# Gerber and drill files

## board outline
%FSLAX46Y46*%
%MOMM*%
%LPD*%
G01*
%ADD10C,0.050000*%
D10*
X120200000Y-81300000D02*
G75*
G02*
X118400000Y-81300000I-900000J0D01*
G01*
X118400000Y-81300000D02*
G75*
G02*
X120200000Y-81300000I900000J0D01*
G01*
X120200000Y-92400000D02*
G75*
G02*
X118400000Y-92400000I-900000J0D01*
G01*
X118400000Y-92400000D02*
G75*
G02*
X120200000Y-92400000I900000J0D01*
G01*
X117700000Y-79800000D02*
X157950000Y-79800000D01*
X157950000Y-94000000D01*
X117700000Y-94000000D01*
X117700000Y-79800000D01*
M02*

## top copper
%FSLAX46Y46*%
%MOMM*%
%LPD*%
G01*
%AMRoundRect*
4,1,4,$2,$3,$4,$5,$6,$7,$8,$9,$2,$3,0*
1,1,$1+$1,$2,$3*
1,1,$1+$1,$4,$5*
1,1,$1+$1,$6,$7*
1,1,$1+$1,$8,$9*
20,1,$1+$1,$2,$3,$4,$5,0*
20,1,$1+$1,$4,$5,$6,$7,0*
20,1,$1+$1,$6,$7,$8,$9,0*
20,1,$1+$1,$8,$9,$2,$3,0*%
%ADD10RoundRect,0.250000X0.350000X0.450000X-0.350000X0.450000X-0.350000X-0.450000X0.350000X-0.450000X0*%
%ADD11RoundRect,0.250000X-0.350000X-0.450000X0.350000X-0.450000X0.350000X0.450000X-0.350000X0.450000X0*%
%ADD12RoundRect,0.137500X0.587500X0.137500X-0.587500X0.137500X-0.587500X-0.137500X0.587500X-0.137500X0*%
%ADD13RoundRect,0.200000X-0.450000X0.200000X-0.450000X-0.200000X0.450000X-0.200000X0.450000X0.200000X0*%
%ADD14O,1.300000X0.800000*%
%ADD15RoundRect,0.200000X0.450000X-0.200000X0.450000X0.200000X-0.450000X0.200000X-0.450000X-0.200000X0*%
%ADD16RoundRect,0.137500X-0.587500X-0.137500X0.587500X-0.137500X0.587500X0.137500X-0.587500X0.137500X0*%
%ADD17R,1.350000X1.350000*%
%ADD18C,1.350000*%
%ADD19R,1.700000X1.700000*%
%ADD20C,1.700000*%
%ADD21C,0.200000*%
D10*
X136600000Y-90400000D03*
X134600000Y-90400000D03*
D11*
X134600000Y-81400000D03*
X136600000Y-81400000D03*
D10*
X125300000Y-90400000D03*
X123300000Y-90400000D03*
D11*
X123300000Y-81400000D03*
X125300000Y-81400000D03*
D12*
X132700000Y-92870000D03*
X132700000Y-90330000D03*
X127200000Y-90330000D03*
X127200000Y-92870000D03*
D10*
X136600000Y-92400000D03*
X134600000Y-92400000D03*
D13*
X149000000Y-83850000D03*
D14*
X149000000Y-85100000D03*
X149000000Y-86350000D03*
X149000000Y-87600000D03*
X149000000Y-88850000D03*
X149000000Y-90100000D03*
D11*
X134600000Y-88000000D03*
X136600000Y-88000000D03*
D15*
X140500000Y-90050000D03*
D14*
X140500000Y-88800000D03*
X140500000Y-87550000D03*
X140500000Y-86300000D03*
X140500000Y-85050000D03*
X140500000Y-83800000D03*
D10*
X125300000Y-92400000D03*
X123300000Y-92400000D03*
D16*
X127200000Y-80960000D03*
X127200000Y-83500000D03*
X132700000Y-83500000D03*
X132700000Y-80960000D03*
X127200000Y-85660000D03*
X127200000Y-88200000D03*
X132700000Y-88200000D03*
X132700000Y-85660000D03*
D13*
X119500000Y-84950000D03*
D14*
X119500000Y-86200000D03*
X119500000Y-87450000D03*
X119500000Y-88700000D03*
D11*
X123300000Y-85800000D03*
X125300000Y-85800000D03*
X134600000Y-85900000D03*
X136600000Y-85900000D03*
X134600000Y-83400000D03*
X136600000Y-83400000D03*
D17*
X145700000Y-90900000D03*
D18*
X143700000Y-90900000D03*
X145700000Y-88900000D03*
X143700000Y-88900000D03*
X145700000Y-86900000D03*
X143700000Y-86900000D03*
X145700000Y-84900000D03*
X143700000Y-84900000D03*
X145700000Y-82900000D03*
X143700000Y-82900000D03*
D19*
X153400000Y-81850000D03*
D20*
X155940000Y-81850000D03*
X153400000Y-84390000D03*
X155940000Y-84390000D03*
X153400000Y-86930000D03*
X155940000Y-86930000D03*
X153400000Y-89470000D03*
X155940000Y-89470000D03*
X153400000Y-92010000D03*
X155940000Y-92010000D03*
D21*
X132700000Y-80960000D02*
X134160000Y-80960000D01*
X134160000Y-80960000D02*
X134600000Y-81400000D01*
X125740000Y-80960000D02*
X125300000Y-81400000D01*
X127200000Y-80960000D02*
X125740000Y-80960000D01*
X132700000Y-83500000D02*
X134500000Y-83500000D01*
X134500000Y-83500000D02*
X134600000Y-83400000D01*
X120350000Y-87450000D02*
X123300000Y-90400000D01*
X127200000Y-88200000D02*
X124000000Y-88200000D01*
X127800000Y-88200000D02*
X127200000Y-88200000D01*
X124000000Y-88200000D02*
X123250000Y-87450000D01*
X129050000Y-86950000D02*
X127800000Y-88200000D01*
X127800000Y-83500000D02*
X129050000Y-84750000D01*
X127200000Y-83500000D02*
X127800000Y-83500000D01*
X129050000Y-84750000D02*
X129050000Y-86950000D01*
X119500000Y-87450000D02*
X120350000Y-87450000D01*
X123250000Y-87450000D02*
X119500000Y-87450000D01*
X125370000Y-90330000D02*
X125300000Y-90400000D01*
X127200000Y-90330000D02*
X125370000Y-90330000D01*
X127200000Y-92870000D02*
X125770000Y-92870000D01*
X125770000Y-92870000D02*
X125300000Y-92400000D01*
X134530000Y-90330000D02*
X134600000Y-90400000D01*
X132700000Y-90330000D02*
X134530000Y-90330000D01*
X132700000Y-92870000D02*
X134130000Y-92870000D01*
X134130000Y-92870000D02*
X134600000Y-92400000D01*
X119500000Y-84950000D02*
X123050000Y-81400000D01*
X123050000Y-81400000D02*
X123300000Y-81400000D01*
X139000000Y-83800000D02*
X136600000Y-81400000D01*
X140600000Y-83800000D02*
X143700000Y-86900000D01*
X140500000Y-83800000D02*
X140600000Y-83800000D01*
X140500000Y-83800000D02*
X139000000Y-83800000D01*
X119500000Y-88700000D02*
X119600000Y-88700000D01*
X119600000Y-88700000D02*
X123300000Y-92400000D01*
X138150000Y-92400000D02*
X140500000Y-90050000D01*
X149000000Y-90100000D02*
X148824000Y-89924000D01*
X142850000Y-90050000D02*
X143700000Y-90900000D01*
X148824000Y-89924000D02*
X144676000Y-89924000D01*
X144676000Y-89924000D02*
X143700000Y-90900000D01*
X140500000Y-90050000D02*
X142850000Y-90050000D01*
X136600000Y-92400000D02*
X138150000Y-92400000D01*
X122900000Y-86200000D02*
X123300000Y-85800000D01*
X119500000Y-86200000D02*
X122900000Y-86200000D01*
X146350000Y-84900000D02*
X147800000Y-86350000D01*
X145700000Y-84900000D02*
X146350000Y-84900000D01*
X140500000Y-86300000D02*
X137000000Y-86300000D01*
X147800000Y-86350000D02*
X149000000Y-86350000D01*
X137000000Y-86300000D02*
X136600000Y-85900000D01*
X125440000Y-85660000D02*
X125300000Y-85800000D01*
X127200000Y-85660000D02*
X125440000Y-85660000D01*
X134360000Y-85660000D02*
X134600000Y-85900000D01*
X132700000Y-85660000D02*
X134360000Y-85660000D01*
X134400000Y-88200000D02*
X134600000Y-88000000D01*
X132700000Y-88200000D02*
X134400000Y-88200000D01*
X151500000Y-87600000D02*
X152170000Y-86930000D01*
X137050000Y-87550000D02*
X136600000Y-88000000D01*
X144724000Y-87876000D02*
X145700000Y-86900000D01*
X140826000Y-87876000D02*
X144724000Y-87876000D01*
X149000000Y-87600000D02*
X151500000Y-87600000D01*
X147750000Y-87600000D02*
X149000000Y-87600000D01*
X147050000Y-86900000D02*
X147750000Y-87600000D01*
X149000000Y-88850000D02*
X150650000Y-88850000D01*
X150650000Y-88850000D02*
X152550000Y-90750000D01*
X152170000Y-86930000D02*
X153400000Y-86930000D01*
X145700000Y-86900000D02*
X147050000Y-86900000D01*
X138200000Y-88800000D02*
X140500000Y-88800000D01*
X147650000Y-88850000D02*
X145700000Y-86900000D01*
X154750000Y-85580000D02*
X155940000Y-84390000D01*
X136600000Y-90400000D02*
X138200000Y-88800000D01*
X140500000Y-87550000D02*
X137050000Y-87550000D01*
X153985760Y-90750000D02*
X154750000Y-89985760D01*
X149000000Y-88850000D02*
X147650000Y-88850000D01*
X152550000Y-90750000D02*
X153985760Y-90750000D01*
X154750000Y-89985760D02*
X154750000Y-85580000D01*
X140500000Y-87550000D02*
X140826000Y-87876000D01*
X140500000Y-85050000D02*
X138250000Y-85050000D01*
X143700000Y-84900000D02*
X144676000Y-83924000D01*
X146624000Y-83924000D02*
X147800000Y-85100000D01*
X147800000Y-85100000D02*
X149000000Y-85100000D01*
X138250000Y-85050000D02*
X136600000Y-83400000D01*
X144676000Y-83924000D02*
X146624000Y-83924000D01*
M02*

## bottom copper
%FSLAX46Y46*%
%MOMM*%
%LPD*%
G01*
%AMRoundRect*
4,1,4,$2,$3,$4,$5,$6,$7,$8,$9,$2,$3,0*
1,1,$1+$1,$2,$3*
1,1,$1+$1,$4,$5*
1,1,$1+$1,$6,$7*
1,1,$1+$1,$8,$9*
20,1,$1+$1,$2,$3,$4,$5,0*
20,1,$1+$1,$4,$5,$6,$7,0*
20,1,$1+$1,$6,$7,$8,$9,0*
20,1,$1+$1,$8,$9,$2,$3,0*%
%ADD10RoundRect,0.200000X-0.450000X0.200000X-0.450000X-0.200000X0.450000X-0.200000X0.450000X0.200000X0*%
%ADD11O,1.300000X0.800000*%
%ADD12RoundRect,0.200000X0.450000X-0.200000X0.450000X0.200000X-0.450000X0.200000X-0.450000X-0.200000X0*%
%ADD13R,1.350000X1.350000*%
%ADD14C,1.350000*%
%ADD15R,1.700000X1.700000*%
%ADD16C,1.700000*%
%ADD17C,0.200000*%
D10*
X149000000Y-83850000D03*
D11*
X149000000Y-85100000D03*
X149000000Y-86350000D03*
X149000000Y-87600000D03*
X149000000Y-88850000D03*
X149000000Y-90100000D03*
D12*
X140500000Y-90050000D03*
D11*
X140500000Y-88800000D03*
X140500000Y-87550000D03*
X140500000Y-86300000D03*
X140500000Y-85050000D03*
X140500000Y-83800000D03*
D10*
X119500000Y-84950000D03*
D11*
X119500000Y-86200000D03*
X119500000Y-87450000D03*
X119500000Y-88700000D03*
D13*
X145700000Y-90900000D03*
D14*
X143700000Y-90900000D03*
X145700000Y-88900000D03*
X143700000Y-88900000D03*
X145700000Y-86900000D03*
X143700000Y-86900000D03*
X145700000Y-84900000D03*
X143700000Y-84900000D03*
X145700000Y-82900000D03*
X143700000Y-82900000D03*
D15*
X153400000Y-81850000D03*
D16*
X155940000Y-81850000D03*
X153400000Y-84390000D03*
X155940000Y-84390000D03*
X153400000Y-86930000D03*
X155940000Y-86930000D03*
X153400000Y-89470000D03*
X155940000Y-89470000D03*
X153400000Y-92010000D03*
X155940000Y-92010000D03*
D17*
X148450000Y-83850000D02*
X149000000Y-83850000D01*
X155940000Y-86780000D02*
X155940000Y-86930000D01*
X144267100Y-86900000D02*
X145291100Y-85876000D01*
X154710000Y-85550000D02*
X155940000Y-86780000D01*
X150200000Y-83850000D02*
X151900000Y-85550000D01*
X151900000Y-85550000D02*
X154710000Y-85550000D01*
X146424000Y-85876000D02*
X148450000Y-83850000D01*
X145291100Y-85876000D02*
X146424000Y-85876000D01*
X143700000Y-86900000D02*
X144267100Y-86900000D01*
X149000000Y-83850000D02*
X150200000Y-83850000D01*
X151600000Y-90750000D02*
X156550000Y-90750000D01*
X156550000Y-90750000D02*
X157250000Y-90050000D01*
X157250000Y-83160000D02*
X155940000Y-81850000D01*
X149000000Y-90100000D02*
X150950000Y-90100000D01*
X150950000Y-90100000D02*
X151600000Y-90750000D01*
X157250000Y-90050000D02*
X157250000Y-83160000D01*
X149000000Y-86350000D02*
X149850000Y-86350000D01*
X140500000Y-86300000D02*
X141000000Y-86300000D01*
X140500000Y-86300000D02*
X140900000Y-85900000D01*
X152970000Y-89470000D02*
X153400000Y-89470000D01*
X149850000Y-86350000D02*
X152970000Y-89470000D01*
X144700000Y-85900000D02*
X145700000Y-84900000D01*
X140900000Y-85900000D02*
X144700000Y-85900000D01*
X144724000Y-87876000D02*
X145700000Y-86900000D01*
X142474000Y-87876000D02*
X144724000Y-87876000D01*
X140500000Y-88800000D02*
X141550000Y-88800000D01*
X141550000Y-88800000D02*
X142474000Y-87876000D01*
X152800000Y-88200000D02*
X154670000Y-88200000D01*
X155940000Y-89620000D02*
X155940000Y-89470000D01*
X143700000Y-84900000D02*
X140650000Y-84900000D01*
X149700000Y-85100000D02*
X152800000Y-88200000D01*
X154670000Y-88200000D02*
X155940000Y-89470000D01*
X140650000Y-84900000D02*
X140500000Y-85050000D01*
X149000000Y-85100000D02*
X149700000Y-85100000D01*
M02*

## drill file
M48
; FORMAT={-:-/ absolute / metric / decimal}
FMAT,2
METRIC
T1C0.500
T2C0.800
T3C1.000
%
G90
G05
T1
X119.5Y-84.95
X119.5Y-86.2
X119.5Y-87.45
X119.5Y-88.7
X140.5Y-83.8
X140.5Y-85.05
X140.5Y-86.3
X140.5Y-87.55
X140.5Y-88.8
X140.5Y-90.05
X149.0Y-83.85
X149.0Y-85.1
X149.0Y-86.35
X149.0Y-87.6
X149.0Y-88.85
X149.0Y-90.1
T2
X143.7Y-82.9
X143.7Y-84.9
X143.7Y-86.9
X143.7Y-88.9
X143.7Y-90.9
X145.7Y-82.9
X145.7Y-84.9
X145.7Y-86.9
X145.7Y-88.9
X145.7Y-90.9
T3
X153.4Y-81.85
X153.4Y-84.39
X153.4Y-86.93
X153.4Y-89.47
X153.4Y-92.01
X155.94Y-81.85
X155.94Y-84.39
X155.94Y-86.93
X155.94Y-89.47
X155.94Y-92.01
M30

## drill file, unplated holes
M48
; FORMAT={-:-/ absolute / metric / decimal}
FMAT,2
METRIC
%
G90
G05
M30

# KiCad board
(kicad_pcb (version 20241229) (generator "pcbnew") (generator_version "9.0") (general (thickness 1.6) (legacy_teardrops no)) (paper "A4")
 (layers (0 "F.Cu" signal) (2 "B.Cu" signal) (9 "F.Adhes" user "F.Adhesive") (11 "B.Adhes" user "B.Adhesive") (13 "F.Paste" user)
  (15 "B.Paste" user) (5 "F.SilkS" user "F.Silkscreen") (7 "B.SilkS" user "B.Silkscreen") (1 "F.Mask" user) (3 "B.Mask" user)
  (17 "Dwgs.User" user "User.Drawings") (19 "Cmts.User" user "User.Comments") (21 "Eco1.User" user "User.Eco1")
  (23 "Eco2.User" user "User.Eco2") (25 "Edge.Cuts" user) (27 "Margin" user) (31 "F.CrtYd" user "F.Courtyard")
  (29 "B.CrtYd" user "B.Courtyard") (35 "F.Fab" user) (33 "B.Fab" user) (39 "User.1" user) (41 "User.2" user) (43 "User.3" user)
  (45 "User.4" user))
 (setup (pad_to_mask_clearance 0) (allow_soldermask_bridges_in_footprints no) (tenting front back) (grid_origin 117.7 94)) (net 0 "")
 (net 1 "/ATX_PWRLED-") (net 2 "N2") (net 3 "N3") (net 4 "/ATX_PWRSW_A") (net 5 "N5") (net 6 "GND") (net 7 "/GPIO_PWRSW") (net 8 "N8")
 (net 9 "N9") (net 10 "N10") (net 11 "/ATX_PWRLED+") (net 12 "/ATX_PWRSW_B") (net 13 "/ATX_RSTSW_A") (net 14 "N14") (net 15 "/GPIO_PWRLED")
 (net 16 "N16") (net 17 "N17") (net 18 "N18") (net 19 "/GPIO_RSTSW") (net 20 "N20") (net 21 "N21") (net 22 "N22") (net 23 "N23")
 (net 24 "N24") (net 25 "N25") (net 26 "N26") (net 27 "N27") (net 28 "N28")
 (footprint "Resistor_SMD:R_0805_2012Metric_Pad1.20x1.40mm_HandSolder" (layer "F.Cu") (at 135.6 90.4 180)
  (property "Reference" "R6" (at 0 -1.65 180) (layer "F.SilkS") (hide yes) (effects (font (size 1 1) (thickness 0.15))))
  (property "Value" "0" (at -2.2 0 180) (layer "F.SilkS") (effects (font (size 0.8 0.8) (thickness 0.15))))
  (pad "1" smd roundrect (at -1 0 180) (size 1.2 1.4) (layers "F.Cu" "F.Mask" "F.Paste") (roundrect_rratio 0.208333) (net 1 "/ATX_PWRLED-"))
  (pad "2" smd roundrect (at 1 0 180) (size 1.2 1.4) (layers "F.Cu" "F.Mask" "F.Paste") (roundrect_rratio 0.208333) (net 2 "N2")))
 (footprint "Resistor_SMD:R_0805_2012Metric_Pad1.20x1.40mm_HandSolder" (layer "F.Cu") (at 135.6 81.4)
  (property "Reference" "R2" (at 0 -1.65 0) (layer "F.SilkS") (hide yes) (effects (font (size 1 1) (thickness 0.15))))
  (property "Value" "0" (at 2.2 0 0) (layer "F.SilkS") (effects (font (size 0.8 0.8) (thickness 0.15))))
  (pad "1" smd roundrect (at -1 0) (size 1.2 1.4) (layers "F.Cu" "F.Mask" "F.Paste") (roundrect_rratio 0.208333) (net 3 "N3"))
  (pad "2" smd roundrect (at 1 0) (size 1.2 1.4) (layers "F.Cu" "F.Mask" "F.Paste") (roundrect_rratio 0.208333) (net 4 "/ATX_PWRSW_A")))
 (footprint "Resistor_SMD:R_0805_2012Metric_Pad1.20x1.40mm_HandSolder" (layer "F.Cu") (at 124.3 90.4 180)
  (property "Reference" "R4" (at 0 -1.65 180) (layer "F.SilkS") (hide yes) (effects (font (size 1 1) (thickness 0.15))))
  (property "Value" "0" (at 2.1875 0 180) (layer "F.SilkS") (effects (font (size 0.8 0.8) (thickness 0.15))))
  (pad "1" smd roundrect (at -1 0 180) (size 1.2 1.4) (layers "F.Cu" "F.Mask" "F.Paste") (roundrect_rratio 0.208333) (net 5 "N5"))
  (pad "2" smd roundrect (at 1 0 180) (size 1.2 1.4) (layers "F.Cu" "F.Mask" "F.Paste") (roundrect_rratio 0.208333) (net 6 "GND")))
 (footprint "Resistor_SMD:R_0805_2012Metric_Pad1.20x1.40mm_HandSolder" (layer "F.Cu") (at 124.3 81.4)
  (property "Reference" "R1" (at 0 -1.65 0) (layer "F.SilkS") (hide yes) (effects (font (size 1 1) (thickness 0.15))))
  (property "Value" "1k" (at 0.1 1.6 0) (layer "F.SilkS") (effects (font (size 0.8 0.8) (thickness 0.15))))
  (pad "1" smd roundrect (at -1 0) (size 1.2 1.4) (layers "F.Cu" "F.Mask" "F.Paste") (roundrect_rratio 0.208333) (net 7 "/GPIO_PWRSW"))
  (pad "2" smd roundrect (at 1 0) (size 1.2 1.4) (layers "F.Cu" "F.Mask" "F.Paste") (roundrect_rratio 0.208333) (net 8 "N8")))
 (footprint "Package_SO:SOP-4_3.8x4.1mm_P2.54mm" (layer "F.Cu") (at 129.95 91.6 180)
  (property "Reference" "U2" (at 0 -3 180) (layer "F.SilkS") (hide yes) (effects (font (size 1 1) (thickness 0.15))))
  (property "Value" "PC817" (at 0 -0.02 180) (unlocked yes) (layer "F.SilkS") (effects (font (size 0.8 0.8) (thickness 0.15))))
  (pad "1" smd roundrect (at -2.75 -1.27 180) (size 1.45 0.55) (layers "F.Cu" "F.Mask" "F.Paste") (roundrect_rratio 0.25) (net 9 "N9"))
  (pad "2" smd roundrect (at -2.75 1.27 180) (size 1.45 0.55) (layers "F.Cu" "F.Mask" "F.Paste") (roundrect_rratio 0.25) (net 2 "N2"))
  (pad "3" smd roundrect (at 2.75 1.27 180) (size 1.45 0.55) (layers "F.Cu" "F.Mask" "F.Paste") (roundrect_rratio 0.25) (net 5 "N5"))
  (pad "4" smd roundrect (at 2.75 -1.27 180) (size 1.45 0.55) (layers "F.Cu" "F.Mask" "F.Paste") (roundrect_rratio 0.25) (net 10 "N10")))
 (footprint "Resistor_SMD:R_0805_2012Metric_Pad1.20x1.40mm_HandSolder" (layer "F.Cu") (at 135.6 92.4 180)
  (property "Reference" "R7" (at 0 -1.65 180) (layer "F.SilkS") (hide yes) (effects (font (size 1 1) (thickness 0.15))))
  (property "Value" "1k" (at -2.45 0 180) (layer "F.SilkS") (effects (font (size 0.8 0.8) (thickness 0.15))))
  (pad "1" smd roundrect (at -1 0 180) (size 1.2 1.4) (layers "F.Cu" "F.Mask" "F.Paste") (roundrect_rratio 0.208333) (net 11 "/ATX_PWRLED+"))
  (pad "2" smd roundrect (at 1 0 180) (size 1.2 1.4) (layers "F.Cu" "F.Mask" "F.Paste") (roundrect_rratio 0.208333) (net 9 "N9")))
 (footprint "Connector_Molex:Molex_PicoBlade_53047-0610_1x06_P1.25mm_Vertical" (layer "F.Cu") (at 149 83.85 -90)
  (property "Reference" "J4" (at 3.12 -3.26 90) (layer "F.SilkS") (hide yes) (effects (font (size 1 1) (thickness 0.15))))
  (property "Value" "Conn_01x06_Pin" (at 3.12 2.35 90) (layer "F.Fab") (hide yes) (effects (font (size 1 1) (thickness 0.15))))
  (pad "1" thru_hole roundrect (at 0 0 270) (size 0.8 1.3) (drill 0.5) (layers "*.Cu" "*.Mask") (remove_unused_layers no)
   (roundrect_rratio 0.25) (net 4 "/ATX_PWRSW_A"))
  (pad "2" thru_hole oval (at 1.25 0 270) (size 0.8 1.3) (drill 0.5) (layers "*.Cu" "*.Mask") (remove_unused_layers no)
   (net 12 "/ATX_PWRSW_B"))
  (pad "3" thru_hole oval (at 2.5 0 270) (size 0.8 1.3) (drill 0.5) (layers "*.Cu" "*.Mask") (remove_unused_layers no)
   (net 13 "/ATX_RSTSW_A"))
  (pad "4" thru_hole oval (at 3.75 0 270) (size 0.8 1.3) (drill 0.5) (layers "*.Cu" "*.Mask") (remove_unused_layers no)
   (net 1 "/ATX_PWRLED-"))
  (pad "5" thru_hole oval (at 5 0 270) (size 0.8 1.3) (drill 0.5) (layers "*.Cu" "*.Mask") (remove_unused_layers no) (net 1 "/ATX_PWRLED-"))
  (pad "6" thru_hole oval (at 6.25 0 270) (size 0.8 1.3) (drill 0.5) (layers "*.Cu" "*.Mask") (remove_unused_layers no)
   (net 11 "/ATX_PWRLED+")))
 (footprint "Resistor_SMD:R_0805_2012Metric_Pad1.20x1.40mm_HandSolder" (layer "F.Cu") (at 135.6 88)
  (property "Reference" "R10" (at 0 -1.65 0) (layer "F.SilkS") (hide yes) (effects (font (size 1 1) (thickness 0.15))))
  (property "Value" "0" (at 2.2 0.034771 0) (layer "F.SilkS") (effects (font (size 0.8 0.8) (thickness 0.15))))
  (pad "1" smd roundrect (at -1 0) (size 1.2 1.4) (layers "F.Cu" "F.Mask" "F.Paste") (roundrect_rratio 0.208333) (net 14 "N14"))
  (pad "2" smd roundrect (at 1 0) (size 1.2 1.4) (layers "F.Cu" "F.Mask" "F.Paste") (roundrect_rratio 0.208333) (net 1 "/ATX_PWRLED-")))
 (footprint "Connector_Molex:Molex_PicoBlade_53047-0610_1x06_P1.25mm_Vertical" (layer "F.Cu") (at 140.5 90.05 90)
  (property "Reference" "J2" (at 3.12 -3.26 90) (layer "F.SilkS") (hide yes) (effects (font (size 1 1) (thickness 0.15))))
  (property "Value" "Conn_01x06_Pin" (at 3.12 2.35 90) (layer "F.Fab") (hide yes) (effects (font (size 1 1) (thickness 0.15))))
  (pad "1" thru_hole roundrect (at 0 0 90) (size 0.8 1.3) (drill 0.5) (layers "*.Cu" "*.Mask") (remove_unused_layers no)
   (roundrect_rratio 0.25) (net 11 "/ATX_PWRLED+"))
  (pad "2" thru_hole oval (at 1.25 0 90) (size 0.8 1.3) (drill 0.5) (layers "*.Cu" "*.Mask") (remove_unused_layers no)
   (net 1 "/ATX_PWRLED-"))
  (pad "3" thru_hole oval (at 2.5 0 90) (size 0.8 1.3) (drill 0.5) (layers "*.Cu" "*.Mask") (remove_unused_layers no) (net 1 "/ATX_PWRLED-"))
  (pad "4" thru_hole oval (at 3.75 0 90) (size 0.8 1.3) (drill 0.5) (layers "*.Cu" "*.Mask") (remove_unused_layers no)
   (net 13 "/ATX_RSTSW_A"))
  (pad "5" thru_hole oval (at 5 0 90) (size 0.8 1.3) (drill 0.5) (layers "*.Cu" "*.Mask") (remove_unused_layers no) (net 12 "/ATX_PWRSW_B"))
  (pad "6" thru_hole oval (at 6.25 0 90) (size 0.8 1.3) (drill 0.5) (layers "*.Cu" "*.Mask") (remove_unused_layers no)
   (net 4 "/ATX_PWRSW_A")))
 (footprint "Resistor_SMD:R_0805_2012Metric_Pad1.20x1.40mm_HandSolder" (layer "F.Cu") (at 124.3 92.4 180)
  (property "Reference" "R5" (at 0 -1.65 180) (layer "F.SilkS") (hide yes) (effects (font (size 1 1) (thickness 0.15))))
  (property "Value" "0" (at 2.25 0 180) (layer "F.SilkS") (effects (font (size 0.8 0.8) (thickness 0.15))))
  (pad "1" smd roundrect (at -1 0 180) (size 1.2 1.4) (layers "F.Cu" "F.Mask" "F.Paste") (roundrect_rratio 0.208333) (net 10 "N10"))
  (pad "2" smd roundrect (at 1 0 180) (size 1.2 1.4) (layers "F.Cu" "F.Mask" "F.Paste") (roundrect_rratio 0.208333) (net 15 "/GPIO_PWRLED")))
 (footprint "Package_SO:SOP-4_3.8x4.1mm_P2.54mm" (layer "F.Cu") (at 129.95 82.23)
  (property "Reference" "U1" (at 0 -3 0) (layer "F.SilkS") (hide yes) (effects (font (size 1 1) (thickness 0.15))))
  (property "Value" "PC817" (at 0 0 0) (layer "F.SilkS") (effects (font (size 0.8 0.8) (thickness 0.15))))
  (pad "1" smd roundrect (at -2.75 -1.27) (size 1.45 0.55) (layers "F.Cu" "F.Mask" "F.Paste") (roundrect_rratio 0.25) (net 8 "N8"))
  (pad "2" smd roundrect (at -2.75 1.27) (size 1.45 0.55) (layers "F.Cu" "F.Mask" "F.Paste") (roundrect_rratio 0.25) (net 6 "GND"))
  (pad "3" smd roundrect (at 2.75 1.27) (size 1.45 0.55) (layers "F.Cu" "F.Mask" "F.Paste") (roundrect_rratio 0.25) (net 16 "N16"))
  (pad "4" smd roundrect (at 2.75 -1.27) (size 1.45 0.55) (layers "F.Cu" "F.Mask" "F.Paste") (roundrect_rratio 0.25) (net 3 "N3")))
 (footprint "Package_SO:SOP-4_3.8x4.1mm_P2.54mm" (layer "F.Cu") (at 129.95 86.93)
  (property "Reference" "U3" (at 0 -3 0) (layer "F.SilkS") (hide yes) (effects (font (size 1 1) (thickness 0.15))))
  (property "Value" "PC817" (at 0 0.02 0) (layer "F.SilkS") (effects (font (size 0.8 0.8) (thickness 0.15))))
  (pad "1" smd roundrect (at -2.75 -1.27) (size 1.45 0.55) (layers "F.Cu" "F.Mask" "F.Paste") (roundrect_rratio 0.25) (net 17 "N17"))
  (pad "2" smd roundrect (at -2.75 1.27) (size 1.45 0.55) (layers "F.Cu" "F.Mask" "F.Paste") (roundrect_rratio 0.25) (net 6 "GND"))
  (pad "3" smd roundrect (at 2.75 1.27) (size 1.45 0.55) (layers "F.Cu" "F.Mask" "F.Paste") (roundrect_rratio 0.25) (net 14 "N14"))
  (pad "4" smd roundrect (at 2.75 -1.27) (size 1.45 0.55) (layers "F.Cu" "F.Mask" "F.Paste") (roundrect_rratio 0.25) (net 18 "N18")))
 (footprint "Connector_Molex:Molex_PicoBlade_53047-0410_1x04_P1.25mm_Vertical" (layer "F.Cu") (at 119.5 84.95 -90)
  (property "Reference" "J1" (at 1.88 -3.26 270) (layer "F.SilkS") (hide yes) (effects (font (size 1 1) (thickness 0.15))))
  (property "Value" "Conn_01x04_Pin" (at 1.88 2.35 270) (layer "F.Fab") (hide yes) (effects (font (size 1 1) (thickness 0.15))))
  (pad "1" thru_hole roundrect (at 0 0 270) (size 0.8 1.3) (drill 0.5) (layers "*.Cu" "*.Mask") (remove_unused_layers no)
   (roundrect_rratio 0.25) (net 7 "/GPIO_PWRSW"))
  (pad "2" thru_hole oval (at 1.25 0 270) (size 0.8 1.3) (drill 0.5) (layers "*.Cu" "*.Mask") (remove_unused_layers no)
   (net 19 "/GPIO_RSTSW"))
  (pad "3" thru_hole oval (at 2.5 0 270) (size 0.8 1.3) (drill 0.5) (layers "*.Cu" "*.Mask") (remove_unused_layers no) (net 6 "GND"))
  (pad "4" thru_hole oval (at 3.75 0 270) (size 0.8 1.3) (drill 0.5) (layers "*.Cu" "*.Mask") (remove_unused_layers no)
   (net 15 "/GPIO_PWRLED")))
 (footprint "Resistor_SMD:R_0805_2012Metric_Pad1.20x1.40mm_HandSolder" (layer "F.Cu") (at 124.3 85.8)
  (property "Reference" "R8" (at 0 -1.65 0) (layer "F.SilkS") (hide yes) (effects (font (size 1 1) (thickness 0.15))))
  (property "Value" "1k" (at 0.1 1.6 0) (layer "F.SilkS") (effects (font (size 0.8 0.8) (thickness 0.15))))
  (pad "1" smd roundrect (at -1 0) (size 1.2 1.4) (layers "F.Cu" "F.Mask" "F.Paste") (roundrect_rratio 0.208333) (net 19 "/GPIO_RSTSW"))
  (pad "2" smd roundrect (at 1 0) (size 1.2 1.4) (layers "F.Cu" "F.Mask" "F.Paste") (roundrect_rratio 0.208333) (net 17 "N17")))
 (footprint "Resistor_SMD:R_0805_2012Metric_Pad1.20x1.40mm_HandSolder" (layer "F.Cu") (at 135.6 85.9)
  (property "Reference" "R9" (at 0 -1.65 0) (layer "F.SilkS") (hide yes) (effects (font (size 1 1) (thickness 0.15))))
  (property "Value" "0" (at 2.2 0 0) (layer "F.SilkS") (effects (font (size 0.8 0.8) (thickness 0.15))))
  (pad "1" smd roundrect (at -1 0) (size 1.2 1.4) (layers "F.Cu" "F.Mask" "F.Paste") (roundrect_rratio 0.208333) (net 18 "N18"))
  (pad "2" smd roundrect (at 1 0) (size 1.2 1.4) (layers "F.Cu" "F.Mask" "F.Paste") (roundrect_rratio 0.208333) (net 13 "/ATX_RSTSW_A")))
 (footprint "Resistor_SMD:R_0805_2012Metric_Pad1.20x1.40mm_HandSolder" (layer "F.Cu") (at 135.6 83.4)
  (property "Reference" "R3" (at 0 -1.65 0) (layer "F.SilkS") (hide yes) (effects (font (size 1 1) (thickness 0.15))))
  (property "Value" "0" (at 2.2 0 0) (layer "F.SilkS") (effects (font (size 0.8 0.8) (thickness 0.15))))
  (pad "1" smd roundrect (at -1 0) (size 1.2 1.4) (layers "F.Cu" "F.Mask" "F.Paste") (roundrect_rratio 0.208333) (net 16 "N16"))
  (pad "2" smd roundrect (at 1 0) (size 1.2 1.4) (layers "F.Cu" "F.Mask" "F.Paste") (roundrect_rratio 0.208333) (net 12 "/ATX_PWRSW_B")))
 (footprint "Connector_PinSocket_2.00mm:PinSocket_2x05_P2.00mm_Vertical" (layer "B.Cu") (at 145.7 90.9)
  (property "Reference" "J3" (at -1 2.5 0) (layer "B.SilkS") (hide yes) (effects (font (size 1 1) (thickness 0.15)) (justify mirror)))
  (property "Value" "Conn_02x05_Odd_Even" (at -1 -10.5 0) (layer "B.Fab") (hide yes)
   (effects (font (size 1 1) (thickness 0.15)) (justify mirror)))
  (pad "1" thru_hole rect (at 0 0) (size 1.35 1.35) (drill 0.8) (layers "*.Cu" "*.Mask") (remove_unused_layers no) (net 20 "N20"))
  (pad "2" thru_hole circle (at -2 0) (size 1.35 1.35) (drill 0.8) (layers "*.Cu" "*.Mask") (remove_unused_layers no)
   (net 11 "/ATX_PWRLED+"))
  (pad "3" thru_hole circle (at 0 -2) (size 1.35 1.35) (drill 0.8) (layers "*.Cu" "*.Mask") (remove_unused_layers no) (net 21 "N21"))
  (pad "4" thru_hole circle (at -2 -2) (size 1.35 1.35) (drill 0.8) (layers "*.Cu" "*.Mask") (remove_unused_layers no) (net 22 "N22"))
  (pad "5" thru_hole circle (at 0 -4) (size 1.35 1.35) (drill 0.8) (layers "*.Cu" "*.Mask") (remove_unused_layers no) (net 1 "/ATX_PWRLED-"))
  (pad "6" thru_hole circle (at -2 -4) (size 1.35 1.35) (drill 0.8) (layers "*.Cu" "*.Mask") (remove_unused_layers no)
   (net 4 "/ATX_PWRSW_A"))
  (pad "7" thru_hole circle (at 0 -6) (size 1.35 1.35) (drill 0.8) (layers "*.Cu" "*.Mask") (remove_unused_layers no)
   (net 13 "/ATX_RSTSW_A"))
  (pad "8" thru_hole circle (at -2 -6) (size 1.35 1.35) (drill 0.8) (layers "*.Cu" "*.Mask") (remove_unused_layers no)
   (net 12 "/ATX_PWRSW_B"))
  (pad "9" thru_hole circle (at 0 -8) (size 1.35 1.35) (drill 0.8) (layers "*.Cu" "*.Mask") (remove_unused_layers no) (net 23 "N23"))
  (pad "10" thru_hole circle (at -2 -8) (size 1.35 1.35) (drill 0.8) (layers "*.Cu" "*.Mask") (remove_unused_layers no) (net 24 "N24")))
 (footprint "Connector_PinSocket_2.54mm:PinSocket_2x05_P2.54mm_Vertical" (layer "B.Cu") (at 153.4 81.85 180)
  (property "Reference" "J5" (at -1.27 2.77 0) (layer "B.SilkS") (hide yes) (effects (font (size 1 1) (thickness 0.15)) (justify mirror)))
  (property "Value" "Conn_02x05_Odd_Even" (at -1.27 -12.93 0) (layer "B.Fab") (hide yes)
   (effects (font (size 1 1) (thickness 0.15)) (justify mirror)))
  (pad "1" thru_hole rect (at 0 0 180) (size 1.7 1.7) (drill 1) (layers "*.Cu" "*.Mask") (remove_unused_layers no) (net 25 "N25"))
  (pad "2" thru_hole circle (at -2.54 0 180) (size 1.7 1.7) (drill 1) (layers "*.Cu" "*.Mask") (remove_unused_layers no)
   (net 11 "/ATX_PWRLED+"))
  (pad "3" thru_hole circle (at 0 -2.54 180) (size 1.7 1.7) (drill 1) (layers "*.Cu" "*.Mask") (remove_unused_layers no) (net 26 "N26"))
  (pad "4" thru_hole circle (at -2.54 -2.54 180) (size 1.7 1.7) (drill 1) (layers "*.Cu" "*.Mask") (remove_unused_layers no)
   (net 1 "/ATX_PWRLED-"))
  (pad "5" thru_hole circle (at 0 -5.08 180) (size 1.7 1.7) (drill 1) (layers "*.Cu" "*.Mask") (remove_unused_layers no)
   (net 1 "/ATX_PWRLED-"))
  (pad "6" thru_hole circle (at -2.54 -5.08 180) (size 1.7 1.7) (drill 1) (layers "*.Cu" "*.Mask") (remove_unused_layers no)
   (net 4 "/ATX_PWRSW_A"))
  (pad "7" thru_hole circle (at 0 -7.62 180) (size 1.7 1.7) (drill 1) (layers "*.Cu" "*.Mask") (remove_unused_layers no)
   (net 13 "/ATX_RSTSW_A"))
  (pad "8" thru_hole circle (at -2.54 -7.62 180) (size 1.7 1.7) (drill 1) (layers "*.Cu" "*.Mask") (remove_unused_layers no)
   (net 12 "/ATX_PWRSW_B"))
  (pad "9" thru_hole circle (at 0 -10.16 180) (size 1.7 1.7) (drill 1) (layers "*.Cu" "*.Mask") (remove_unused_layers no) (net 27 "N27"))
  (pad "10" thru_hole circle (at -2.54 -10.16 180) (size 1.7 1.7) (drill 1) (layers "*.Cu" "*.Mask") (remove_unused_layers no)
   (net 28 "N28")))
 (gr_circle (center 119.3 81.3) (end 120.2 81.3) (stroke (width 0.05) (type solid)) (fill no) (layer "Edge.Cuts"))
 (gr_circle (center 119.3 92.4) (end 120.2 92.4) (stroke (width 0.05) (type solid)) (fill no) (layer "Edge.Cuts"))
 (gr_rect (start 117.7 79.8) (end 157.95 94) (stroke (width 0.05) (type default)) (fill no) (layer "Edge.Cuts"))
 (segment (start 132.7 80.96) (end 134.16 80.96) (width 0.2) (layer "F.Cu") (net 3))
 (segment (start 134.16 80.96) (end 134.6 81.4) (width 0.2) (layer "F.Cu") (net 3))
 (segment (start 125.74 80.96) (end 125.3 81.4) (width 0.2) (layer "F.Cu") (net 8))
 (segment (start 127.2 80.96) (end 125.74 80.96) (width 0.2) (layer "F.Cu") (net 8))
 (segment (start 132.7 83.5) (end 134.5 83.5) (width 0.2) (layer "F.Cu") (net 16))
 (segment (start 134.5 83.5) (end 134.6 83.4) (width 0.2) (layer "F.Cu") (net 16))
 (segment (start 120.35 87.45) (end 123.3 90.4) (width 0.2) (layer "F.Cu") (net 6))
 (segment (start 127.2 88.2) (end 124 88.2) (width 0.2) (layer "F.Cu") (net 6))
 (segment (start 127.8 88.2) (end 127.2 88.2) (width 0.2) (layer "F.Cu") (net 6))
 (segment (start 124 88.2) (end 123.25 87.45) (width 0.2) (layer "F.Cu") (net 6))
 (segment (start 129.05 86.95) (end 127.8 88.2) (width 0.2) (layer "F.Cu") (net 6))
 (segment (start 127.8 83.5) (end 129.05 84.75) (width 0.2) (layer "F.Cu") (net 6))
 (segment (start 127.2 83.5) (end 127.8 83.5) (width 0.2) (layer "F.Cu") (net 6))
 (segment (start 129.05 84.75) (end 129.05 86.95) (width 0.2) (layer "F.Cu") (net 6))
 (segment (start 119.5 87.45) (end 120.35 87.45) (width 0.2) (layer "F.Cu") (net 6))
 (segment (start 123.25 87.45) (end 119.5 87.45) (width 0.2) (layer "F.Cu") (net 6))
 (segment (start 125.37 90.33) (end 125.3 90.4) (width 0.2) (layer "F.Cu") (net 5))
 (segment (start 127.2 90.33) (end 125.37 90.33) (width 0.2) (layer "F.Cu") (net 5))
 (segment (start 127.2 92.87) (end 125.77 92.87) (width 0.2) (layer "F.Cu") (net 10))
 (segment (start 125.77 92.87) (end 125.3 92.4) (width 0.2) (layer "F.Cu") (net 10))
 (segment (start 134.53 90.33) (end 134.6 90.4) (width 0.2) (layer "F.Cu") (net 2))
 (segment (start 132.7 90.33) (end 134.53 90.33) (width 0.2) (layer "F.Cu") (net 2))
 (segment (start 132.7 92.87) (end 134.13 92.87) (width 0.2) (layer "F.Cu") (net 9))
 (segment (start 134.13 92.87) (end 134.6 92.4) (width 0.2) (layer "F.Cu") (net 9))
 (segment (start 119.5 84.95) (end 123.05 81.4) (width 0.2) (layer "F.Cu") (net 7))
 (segment (start 123.05 81.4) (end 123.3 81.4) (width 0.2) (layer "F.Cu") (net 7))
 (segment (start 139 83.8) (end 136.6 81.4) (width 0.2) (layer "F.Cu") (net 4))
 (segment (start 140.6 83.8) (end 143.7 86.9) (width 0.2) (layer "F.Cu") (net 4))
 (segment (start 140.5 83.8) (end 140.6 83.8) (width 0.2) (layer "F.Cu") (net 4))
 (segment (start 140.5 83.8) (end 139 83.8) (width 0.2) (layer "F.Cu") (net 4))
 (segment (start 148.45 83.85) (end 149 83.85) (width 0.2) (layer "B.Cu") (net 4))
 (segment (start 155.94 86.78) (end 155.94 86.93) (width 0.2) (layer "B.Cu") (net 4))
 (segment (start 144.2671 86.9) (end 145.2911 85.876) (width 0.2) (layer "B.Cu") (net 4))
 (segment (start 154.71 85.55) (end 155.94 86.78) (width 0.2) (layer "B.Cu") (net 4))
 (segment (start 150.2 83.85) (end 151.9 85.55) (width 0.2) (layer "B.Cu") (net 4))
 (segment (start 151.9 85.55) (end 154.71 85.55) (width 0.2) (layer "B.Cu") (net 4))
 (segment (start 146.424 85.876) (end 148.45 83.85) (width 0.2) (layer "B.Cu") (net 4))
 (segment (start 145.2911 85.876) (end 146.424 85.876) (width 0.2) (layer "B.Cu") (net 4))
 (segment (start 143.7 86.9) (end 144.2671 86.9) (width 0.2) (layer "B.Cu") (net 4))
 (segment (start 149 83.85) (end 150.2 83.85) (width 0.2) (layer "B.Cu") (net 4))
 (segment (start 119.5 88.7) (end 119.6 88.7) (width 0.2) (layer "F.Cu") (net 15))
 (segment (start 119.6 88.7) (end 123.3 92.4) (width 0.2) (layer "F.Cu") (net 15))
 (segment (start 138.15 92.4) (end 140.5 90.05) (width 0.2) (layer "F.Cu") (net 11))
 (segment (start 149 90.1) (end 148.824 89.924) (width 0.2) (layer "F.Cu") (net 11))
 (segment (start 142.85 90.05) (end 143.7 90.9) (width 0.2) (layer "F.Cu") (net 11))
 (segment (start 148.824 89.924) (end 144.676 89.924) (width 0.2) (layer "F.Cu") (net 11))
 (segment (start 144.676 89.924) (end 143.7 90.9) (width 0.2) (layer "F.Cu") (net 11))
 (segment (start 140.5 90.05) (end 142.85 90.05) (width 0.2) (layer "F.Cu") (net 11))
 (segment (start 136.6 92.4) (end 138.15 92.4) (width 0.2) (layer "F.Cu") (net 11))
 (segment (start 151.6 90.75) (end 156.55 90.75) (width 0.2) (layer "B.Cu") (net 11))
 (segment (start 156.55 90.75) (end 157.25 90.05) (width 0.2) (layer "B.Cu") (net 11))
 (segment (start 157.25 83.16) (end 155.94 81.85) (width 0.2) (layer "B.Cu") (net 11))
 (segment (start 149 90.1) (end 150.95 90.1) (width 0.2) (layer "B.Cu") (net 11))
 (segment (start 150.95 90.1) (end 151.6 90.75) (width 0.2) (layer "B.Cu") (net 11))
 (segment (start 157.25 90.05) (end 157.25 83.16) (width 0.2) (layer "B.Cu") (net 11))
 (segment (start 122.9 86.2) (end 123.3 85.8) (width 0.2) (layer "F.Cu") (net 19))
 (segment (start 119.5 86.2) (end 122.9 86.2) (width 0.2) (layer "F.Cu") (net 19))
 (segment (start 146.35 84.9) (end 147.8 86.35) (width 0.2) (layer "F.Cu") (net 13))
 (segment (start 145.7 84.9) (end 146.35 84.9) (width 0.2) (layer "F.Cu") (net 13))
 (segment (start 140.5 86.3) (end 137 86.3) (width 0.2) (layer "F.Cu") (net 13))
 (segment (start 147.8 86.35) (end 149 86.35) (width 0.2) (layer "F.Cu") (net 13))
 (segment (start 137 86.3) (end 136.6 85.9) (width 0.2) (layer "F.Cu") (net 13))
 (segment (start 149 86.35) (end 149.85 86.35) (width 0.2) (layer "B.Cu") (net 13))
 (segment (start 140.5 86.3) (end 141 86.3) (width 0.2) (layer "B.Cu") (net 13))
 (segment (start 140.5 86.3) (end 140.9 85.9) (width 0.2) (layer "B.Cu") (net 13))
 (segment (start 152.97 89.47) (end 153.4 89.47) (width 0.2) (layer "B.Cu") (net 13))
 (segment (start 149.85 86.35) (end 152.97 89.47) (width 0.2) (layer "B.Cu") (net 13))
 (segment (start 144.7 85.9) (end 145.7 84.9) (width 0.2) (layer "B.Cu") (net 13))
 (segment (start 140.9 85.9) (end 144.7 85.9) (width 0.2) (layer "B.Cu") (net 13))
 (segment (start 125.44 85.66) (end 125.3 85.8) (width 0.2) (layer "F.Cu") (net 17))
 (segment (start 127.2 85.66) (end 125.44 85.66) (width 0.2) (layer "F.Cu") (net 17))
 (segment (start 134.36 85.66) (end 134.6 85.9) (width 0.2) (layer "F.Cu") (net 18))
 (segment (start 132.7 85.66) (end 134.36 85.66) (width 0.2) (layer "F.Cu") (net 18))
 (segment (start 134.4 88.2) (end 134.6 88) (width 0.2) (layer "F.Cu") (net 14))
 (segment (start 132.7 88.2) (end 134.4 88.2) (width 0.2) (layer "F.Cu") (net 14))
 (segment (start 151.5 87.6) (end 152.17 86.93) (width 0.2) (layer "F.Cu") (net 1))
 (segment (start 137.05 87.55) (end 136.6 88) (width 0.2) (layer "F.Cu") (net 1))
 (segment (start 144.724 87.876) (end 145.7 86.9) (width 0.2) (layer "F.Cu") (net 1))
 (segment (start 140.826 87.876) (end 144.724 87.876) (width 0.2) (layer "F.Cu") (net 1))
 (segment (start 149 87.6) (end 151.5 87.6) (width 0.2) (layer "F.Cu") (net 1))
 (segment (start 147.75 87.6) (end 149 87.6) (width 0.2) (layer "F.Cu") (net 1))
 (segment (start 147.05 86.9) (end 147.75 87.6) (width 0.2) (layer "F.Cu") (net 1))
 (segment (start 149 88.85) (end 150.65 88.85) (width 0.2) (layer "F.Cu") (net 1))
 (segment (start 150.65 88.85) (end 152.55 90.75) (width 0.2) (layer "F.Cu") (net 1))
 (segment (start 152.17 86.93) (end 153.4 86.93) (width 0.2) (layer "F.Cu") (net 1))
 (segment (start 145.7 86.9) (end 147.05 86.9) (width 0.2) (layer "F.Cu") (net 1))
 (segment (start 138.2 88.8) (end 140.5 88.8) (width 0.2) (layer "F.Cu") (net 1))
 (segment (start 147.65 88.85) (end 145.7 86.9) (width 0.2) (layer "F.Cu") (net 1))
 (segment (start 154.75 85.58) (end 155.94 84.39) (width 0.2) (layer "F.Cu") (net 1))
 (segment (start 136.6 90.4) (end 138.2 88.8) (width 0.2) (layer "F.Cu") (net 1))
 (segment (start 140.5 87.55) (end 137.05 87.55) (width 0.2) (layer "F.Cu") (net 1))
 (segment (start 153.98576 90.75) (end 154.75 89.98576) (width 0.2) (layer "F.Cu") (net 1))
 (segment (start 149 88.85) (end 147.65 88.85) (width 0.2) (layer "F.Cu") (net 1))
 (segment (start 152.55 90.75) (end 153.98576 90.75) (width 0.2) (layer "F.Cu") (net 1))
 (segment (start 154.75 89.98576) (end 154.75 85.58) (width 0.2) (layer "F.Cu") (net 1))
 (segment (start 140.5 87.55) (end 140.826 87.876) (width 0.2) (layer "F.Cu") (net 1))
 (segment (start 144.724 87.876) (end 145.7 86.9) (width 0.2) (layer "B.Cu") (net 1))
 (segment (start 142.474 87.876) (end 144.724 87.876) (width 0.2) (layer "B.Cu") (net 1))
 (segment (start 140.5 88.8) (end 141.55 88.8) (width 0.2) (layer "B.Cu") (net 1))
 (segment (start 141.55 88.8) (end 142.474 87.876) (width 0.2) (layer "B.Cu") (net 1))
 (segment (start 140.5 85.05) (end 138.25 85.05) (width 0.2) (layer "F.Cu") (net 12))
 (segment (start 143.7 84.9) (end 144.676 83.924) (width 0.2) (layer "F.Cu") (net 12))
 (segment (start 146.624 83.924) (end 147.8 85.1) (width 0.2) (layer "F.Cu") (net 12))
 (segment (start 147.8 85.1) (end 149 85.1) (width 0.2) (layer "F.Cu") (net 12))
 (segment (start 138.25 85.05) (end 136.6 83.4) (width 0.2) (layer "F.Cu") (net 12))
 (segment (start 144.676 83.924) (end 146.624 83.924) (width 0.2) (layer "F.Cu") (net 12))
 (segment (start 152.8 88.2) (end 154.67 88.2) (width 0.2) (layer "B.Cu") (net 12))
 (segment (start 155.94 89.62) (end 155.94 89.47) (width 0.2) (layer "B.Cu") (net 12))
 (segment (start 143.7 84.9) (end 140.65 84.9) (width 0.2) (layer "B.Cu") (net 12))
 (segment (start 149.7 85.1) (end 152.8 88.2) (width 0.2) (layer "B.Cu") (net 12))
 (segment (start 154.67 88.2) (end 155.94 89.47) (width 0.2) (layer "B.Cu") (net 12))
 (segment (start 140.65 84.9) (end 140.5 85.05) (width 0.2) (layer "B.Cu") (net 12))
 (segment (start 149 85.1) (end 149.7 85.1) (width 0.2) (layer "B.Cu") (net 12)))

